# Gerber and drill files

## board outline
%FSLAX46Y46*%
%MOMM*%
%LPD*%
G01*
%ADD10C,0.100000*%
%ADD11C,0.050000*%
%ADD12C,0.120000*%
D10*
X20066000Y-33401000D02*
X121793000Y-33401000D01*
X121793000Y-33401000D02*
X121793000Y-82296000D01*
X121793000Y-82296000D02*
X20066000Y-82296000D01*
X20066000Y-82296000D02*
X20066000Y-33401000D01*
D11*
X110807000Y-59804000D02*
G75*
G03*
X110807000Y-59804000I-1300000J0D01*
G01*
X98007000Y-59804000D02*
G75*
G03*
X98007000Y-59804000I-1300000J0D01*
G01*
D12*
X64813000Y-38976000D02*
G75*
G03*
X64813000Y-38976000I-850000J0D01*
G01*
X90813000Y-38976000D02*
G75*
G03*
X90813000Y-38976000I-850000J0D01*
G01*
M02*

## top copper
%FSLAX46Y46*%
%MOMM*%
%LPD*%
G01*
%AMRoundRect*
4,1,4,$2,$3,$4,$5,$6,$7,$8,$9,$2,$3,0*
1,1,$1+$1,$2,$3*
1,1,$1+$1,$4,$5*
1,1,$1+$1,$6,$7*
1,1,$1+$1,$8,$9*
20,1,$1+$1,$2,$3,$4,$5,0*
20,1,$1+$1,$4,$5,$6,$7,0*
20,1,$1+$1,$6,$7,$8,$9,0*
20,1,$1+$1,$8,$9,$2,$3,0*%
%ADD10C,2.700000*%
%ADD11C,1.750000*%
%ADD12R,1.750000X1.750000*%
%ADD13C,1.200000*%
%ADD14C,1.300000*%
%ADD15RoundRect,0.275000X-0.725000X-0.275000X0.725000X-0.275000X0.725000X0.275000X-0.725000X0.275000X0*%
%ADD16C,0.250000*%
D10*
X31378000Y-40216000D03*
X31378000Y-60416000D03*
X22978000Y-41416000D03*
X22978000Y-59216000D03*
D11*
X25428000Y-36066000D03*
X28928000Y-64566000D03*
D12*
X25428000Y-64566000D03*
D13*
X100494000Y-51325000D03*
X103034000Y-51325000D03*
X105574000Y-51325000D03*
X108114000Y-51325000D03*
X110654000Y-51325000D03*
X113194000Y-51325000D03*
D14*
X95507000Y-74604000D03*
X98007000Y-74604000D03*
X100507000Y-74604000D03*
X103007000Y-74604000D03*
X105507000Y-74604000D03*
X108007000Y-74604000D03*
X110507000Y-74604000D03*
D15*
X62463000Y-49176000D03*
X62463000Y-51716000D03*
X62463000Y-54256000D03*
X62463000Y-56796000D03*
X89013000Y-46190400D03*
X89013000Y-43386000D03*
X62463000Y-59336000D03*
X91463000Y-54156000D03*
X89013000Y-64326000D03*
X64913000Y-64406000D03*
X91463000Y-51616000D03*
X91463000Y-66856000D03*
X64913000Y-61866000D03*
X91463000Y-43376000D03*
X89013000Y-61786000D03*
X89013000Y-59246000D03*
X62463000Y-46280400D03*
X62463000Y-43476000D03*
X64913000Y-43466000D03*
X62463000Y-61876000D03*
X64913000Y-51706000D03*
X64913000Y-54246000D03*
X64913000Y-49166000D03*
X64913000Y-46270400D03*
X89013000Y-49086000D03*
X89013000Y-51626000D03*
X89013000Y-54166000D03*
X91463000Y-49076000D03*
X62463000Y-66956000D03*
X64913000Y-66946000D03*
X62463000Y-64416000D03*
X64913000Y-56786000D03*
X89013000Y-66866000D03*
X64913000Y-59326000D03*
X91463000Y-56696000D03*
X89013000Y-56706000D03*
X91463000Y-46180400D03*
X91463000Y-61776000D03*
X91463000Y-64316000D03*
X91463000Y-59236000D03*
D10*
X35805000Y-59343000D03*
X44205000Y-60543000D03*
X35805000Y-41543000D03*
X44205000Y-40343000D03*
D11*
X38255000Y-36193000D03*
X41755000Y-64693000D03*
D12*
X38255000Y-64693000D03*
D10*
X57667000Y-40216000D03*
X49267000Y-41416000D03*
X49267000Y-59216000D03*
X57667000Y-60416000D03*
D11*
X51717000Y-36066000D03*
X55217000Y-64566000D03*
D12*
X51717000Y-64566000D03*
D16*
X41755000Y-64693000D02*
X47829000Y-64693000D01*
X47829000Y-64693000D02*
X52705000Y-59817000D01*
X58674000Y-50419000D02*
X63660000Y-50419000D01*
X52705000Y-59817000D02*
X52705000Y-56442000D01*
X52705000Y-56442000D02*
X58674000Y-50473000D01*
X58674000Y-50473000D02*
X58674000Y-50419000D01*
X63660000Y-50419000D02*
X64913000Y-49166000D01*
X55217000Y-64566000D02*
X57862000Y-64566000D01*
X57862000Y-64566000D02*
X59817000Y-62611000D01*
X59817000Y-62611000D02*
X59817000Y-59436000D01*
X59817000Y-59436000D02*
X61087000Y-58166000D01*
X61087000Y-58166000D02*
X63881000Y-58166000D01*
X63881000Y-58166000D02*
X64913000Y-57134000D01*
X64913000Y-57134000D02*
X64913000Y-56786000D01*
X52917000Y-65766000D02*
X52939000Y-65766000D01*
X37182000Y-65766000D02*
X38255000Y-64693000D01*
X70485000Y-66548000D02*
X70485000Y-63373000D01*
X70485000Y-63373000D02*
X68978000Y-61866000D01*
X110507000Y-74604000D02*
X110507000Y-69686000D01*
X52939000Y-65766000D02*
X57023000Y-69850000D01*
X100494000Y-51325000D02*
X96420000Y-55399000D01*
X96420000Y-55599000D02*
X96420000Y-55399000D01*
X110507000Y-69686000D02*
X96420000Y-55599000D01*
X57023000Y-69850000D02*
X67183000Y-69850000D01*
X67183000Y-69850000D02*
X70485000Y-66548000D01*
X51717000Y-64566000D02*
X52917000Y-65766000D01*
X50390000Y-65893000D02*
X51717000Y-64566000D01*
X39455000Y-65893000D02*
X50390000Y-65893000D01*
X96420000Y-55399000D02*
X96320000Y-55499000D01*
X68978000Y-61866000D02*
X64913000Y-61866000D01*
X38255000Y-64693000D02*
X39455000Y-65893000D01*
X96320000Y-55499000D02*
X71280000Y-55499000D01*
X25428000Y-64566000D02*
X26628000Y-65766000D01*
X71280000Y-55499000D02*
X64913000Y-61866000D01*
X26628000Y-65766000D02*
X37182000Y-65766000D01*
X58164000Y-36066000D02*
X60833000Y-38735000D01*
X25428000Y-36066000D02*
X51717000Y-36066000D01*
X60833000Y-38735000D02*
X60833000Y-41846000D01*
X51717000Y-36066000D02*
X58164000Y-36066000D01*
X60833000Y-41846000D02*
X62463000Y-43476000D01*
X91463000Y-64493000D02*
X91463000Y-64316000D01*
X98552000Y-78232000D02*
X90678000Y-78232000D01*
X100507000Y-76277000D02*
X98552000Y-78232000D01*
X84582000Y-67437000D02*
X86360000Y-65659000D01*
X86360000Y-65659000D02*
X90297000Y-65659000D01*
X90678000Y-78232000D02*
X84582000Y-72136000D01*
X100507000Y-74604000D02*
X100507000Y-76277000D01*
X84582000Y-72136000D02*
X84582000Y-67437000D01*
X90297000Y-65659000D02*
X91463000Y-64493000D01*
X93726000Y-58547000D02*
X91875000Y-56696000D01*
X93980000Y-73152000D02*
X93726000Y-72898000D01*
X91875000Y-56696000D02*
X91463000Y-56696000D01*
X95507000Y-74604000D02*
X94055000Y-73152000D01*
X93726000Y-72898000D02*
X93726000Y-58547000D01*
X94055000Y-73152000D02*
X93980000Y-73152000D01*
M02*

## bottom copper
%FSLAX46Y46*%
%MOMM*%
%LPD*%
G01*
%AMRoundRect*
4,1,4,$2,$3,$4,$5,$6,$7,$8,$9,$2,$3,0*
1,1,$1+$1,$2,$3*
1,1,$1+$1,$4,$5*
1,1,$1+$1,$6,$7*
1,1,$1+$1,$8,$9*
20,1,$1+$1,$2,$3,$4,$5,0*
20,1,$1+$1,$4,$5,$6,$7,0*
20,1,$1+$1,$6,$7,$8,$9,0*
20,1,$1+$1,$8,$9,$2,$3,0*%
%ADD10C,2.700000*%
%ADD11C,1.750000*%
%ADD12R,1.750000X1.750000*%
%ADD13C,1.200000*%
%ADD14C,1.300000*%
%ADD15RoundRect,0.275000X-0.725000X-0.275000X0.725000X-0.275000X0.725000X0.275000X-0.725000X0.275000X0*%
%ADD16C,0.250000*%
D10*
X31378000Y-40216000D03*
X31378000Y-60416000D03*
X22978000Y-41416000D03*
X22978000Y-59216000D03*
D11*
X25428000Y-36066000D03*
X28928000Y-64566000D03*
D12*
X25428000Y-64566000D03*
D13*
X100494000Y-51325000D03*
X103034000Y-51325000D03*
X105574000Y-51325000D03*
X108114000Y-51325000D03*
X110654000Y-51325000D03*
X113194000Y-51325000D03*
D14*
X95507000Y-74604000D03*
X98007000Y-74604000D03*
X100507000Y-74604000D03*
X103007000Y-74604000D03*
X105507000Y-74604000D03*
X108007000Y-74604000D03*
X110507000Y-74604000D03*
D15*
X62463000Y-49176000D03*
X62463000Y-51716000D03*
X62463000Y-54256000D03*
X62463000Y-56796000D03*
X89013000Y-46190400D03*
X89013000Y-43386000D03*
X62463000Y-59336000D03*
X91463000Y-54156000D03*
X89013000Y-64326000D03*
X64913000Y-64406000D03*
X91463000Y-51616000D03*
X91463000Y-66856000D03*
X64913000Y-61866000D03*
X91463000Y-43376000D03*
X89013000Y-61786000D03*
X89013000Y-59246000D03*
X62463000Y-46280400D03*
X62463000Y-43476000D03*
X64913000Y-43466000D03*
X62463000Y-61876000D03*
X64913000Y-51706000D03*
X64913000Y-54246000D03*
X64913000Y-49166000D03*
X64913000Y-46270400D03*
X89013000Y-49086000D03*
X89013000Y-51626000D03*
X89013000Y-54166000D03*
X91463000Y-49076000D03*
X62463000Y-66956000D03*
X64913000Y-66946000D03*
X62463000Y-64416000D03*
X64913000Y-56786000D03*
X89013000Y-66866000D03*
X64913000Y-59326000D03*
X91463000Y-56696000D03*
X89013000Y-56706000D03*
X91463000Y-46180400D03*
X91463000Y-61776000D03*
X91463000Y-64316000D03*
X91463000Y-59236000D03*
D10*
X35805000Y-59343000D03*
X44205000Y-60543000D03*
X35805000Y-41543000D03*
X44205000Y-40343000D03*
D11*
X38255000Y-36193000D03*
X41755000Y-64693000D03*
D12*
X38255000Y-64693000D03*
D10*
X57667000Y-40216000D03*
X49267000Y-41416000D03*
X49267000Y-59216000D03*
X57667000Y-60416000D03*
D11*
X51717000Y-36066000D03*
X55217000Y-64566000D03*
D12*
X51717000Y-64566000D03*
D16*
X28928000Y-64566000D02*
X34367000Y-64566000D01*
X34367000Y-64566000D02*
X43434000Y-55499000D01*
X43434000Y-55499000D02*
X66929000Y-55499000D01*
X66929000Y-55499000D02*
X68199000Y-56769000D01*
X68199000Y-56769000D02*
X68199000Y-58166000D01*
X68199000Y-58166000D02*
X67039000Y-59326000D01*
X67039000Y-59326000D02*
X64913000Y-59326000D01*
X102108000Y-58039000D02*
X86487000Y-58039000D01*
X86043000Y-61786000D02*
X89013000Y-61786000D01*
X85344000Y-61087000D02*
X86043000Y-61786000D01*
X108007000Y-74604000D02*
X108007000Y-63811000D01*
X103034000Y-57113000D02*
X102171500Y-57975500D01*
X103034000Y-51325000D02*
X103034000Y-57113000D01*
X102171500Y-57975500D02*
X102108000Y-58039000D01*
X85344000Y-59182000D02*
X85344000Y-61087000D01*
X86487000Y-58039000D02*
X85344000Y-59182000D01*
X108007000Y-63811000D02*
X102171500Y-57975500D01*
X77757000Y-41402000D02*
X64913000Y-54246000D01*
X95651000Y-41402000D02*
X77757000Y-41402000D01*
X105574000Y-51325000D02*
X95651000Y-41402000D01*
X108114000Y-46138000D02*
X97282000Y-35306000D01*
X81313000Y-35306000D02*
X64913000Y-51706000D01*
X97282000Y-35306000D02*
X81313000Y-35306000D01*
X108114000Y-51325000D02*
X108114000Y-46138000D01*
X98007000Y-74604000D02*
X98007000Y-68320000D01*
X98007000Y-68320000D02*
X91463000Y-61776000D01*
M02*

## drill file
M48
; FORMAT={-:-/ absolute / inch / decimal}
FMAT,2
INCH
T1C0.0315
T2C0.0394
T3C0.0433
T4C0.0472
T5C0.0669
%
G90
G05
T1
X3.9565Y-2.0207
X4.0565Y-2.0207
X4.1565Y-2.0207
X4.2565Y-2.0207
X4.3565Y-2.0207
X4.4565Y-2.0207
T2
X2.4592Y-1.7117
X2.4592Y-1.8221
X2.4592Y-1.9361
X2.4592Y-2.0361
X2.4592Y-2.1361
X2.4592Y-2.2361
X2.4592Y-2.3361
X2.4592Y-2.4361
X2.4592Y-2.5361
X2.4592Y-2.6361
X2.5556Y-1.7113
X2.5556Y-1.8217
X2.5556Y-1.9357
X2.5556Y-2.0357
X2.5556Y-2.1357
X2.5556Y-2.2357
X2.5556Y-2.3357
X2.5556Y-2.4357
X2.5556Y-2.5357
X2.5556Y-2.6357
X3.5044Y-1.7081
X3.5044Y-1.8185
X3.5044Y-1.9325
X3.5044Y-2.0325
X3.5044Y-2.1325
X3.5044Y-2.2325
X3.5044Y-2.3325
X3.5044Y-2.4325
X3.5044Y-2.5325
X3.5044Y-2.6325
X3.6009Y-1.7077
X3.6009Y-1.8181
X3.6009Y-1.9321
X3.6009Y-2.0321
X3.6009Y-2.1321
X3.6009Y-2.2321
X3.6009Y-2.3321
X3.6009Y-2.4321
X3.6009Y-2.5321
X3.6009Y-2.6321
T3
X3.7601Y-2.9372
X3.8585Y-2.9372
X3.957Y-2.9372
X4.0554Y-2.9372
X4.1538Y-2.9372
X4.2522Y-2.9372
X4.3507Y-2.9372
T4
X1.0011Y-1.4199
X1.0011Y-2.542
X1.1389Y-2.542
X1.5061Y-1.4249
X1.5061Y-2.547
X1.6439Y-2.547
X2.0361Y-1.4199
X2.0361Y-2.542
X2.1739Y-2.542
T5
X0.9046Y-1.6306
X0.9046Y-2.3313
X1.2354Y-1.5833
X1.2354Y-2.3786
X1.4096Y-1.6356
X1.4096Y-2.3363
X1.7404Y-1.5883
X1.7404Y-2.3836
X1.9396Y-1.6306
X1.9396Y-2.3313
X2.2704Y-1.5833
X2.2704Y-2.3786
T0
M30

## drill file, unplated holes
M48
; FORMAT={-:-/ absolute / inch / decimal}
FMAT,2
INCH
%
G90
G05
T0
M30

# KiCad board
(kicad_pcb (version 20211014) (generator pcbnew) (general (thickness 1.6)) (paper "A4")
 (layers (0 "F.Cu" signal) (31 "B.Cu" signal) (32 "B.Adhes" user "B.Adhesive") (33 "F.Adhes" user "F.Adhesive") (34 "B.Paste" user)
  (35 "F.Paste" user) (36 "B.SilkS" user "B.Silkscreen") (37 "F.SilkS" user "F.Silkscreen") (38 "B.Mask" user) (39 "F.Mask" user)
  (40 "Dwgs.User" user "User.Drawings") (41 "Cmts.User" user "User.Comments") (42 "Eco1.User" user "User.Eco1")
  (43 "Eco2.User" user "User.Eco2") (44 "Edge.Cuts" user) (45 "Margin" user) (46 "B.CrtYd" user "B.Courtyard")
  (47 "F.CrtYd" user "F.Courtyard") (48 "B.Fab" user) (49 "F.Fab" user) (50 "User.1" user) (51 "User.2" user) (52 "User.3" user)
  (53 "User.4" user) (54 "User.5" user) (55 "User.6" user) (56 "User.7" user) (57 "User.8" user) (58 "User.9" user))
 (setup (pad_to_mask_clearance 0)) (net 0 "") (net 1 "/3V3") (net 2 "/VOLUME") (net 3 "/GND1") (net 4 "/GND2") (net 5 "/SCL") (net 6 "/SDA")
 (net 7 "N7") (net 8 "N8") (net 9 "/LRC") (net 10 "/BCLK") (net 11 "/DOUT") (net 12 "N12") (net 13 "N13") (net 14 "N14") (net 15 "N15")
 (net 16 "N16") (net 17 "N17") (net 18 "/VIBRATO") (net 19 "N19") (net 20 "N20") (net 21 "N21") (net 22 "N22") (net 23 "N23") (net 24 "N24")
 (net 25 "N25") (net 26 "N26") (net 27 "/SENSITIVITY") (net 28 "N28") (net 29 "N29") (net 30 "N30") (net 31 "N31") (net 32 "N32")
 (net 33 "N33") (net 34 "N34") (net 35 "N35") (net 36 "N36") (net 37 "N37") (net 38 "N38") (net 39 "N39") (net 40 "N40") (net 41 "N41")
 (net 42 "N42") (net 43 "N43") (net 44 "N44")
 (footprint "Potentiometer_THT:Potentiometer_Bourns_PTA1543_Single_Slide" (layer "F.Cu") (at 25.428 64.566 90)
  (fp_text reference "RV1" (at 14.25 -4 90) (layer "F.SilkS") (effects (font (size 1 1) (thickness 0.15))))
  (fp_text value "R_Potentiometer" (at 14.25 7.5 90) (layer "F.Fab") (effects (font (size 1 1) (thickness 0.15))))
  (pad "1" thru_hole rect (at 0 0 90) (size 1.75 1.75) (drill 1.2) (layers *.Cu *.Mask) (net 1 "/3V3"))
  (pad "2" thru_hole circle (at 0 3.5 90) (size 1.75 1.75) (drill 1.2) (layers *.Cu *.Mask) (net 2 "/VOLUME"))
  (pad "3" thru_hole circle (at 28.5 0 90) (size 1.75 1.75) (drill 1.2) (layers *.Cu *.Mask) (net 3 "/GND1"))
  (pad "MP" thru_hole circle (at 5.35 -2.45 90) (size 2.7 2.7) (drill 1.7) (layers *.Cu *.Mask))
  (pad "MP" thru_hole circle (at 23.15 -2.45 90) (size 2.7 2.7) (drill 1.7) (layers *.Cu *.Mask))
  (pad "MP" thru_hole circle (at 4.15 5.95 90) (size 2.7 2.7) (drill 1.7) (layers *.Cu *.Mask))
  (pad "MP" thru_hole circle (at 24.35 5.95 90) (size 2.7 2.7) (drill 1.7) (layers *.Cu *.Mask)))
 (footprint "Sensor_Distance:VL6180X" (layer "F.Cu") (at 94.144 36.085)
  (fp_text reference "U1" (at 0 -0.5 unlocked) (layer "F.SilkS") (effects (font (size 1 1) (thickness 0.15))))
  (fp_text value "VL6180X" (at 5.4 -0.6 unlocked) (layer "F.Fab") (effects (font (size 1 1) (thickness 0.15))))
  (pad "1" thru_hole circle (at 6.35 15.24) (size 1.2 1.2) (drill 0.8) (layers *.Cu *.Mask) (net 1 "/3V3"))
  (pad "2" thru_hole circle (at 8.89 15.24) (size 1.2 1.2) (drill 0.8) (layers *.Cu *.Mask) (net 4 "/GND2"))
  (pad "3" thru_hole circle (at 11.43 15.24) (size 1.2 1.2) (drill 0.8) (layers *.Cu *.Mask) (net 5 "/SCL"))
  (pad "4" thru_hole circle (at 13.97 15.24) (size 1.2 1.2) (drill 0.8) (layers *.Cu *.Mask) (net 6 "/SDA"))
  (pad "5" thru_hole circle (at 16.51 15.24) (size 1.2 1.2) (drill 0.8) (layers *.Cu *.Mask) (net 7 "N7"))
  (pad "6" thru_hole circle (at 19.05 15.24) (size 1.2 1.2) (drill 0.8) (layers *.Cu *.Mask) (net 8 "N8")))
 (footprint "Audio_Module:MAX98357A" (layer "F.Cu") (at 94.107 57.404)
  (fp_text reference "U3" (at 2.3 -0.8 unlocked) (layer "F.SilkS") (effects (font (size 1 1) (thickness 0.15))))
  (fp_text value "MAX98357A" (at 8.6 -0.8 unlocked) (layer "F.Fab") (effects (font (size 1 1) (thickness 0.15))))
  (fp_circle (center 15.4 2.4) (end 16.7 2.4) (layer "Edge.Cuts") (width 0.05) (fill none))
  (fp_circle (center 2.6 2.4) (end 3.9 2.4) (layer "Edge.Cuts") (width 0.05) (fill none))
  (pad "1" thru_hole circle (at 1.4 17.2) (size 1.3 1.3) (drill 1.1) (layers *.Cu *.Mask) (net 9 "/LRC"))
  (pad "2" thru_hole circle (at 3.9 17.2) (size 1.3 1.3) (drill 1.1) (layers *.Cu *.Mask) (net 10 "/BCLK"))
  (pad "3" thru_hole circle (at 6.4 17.2) (size 1.3 1.3) (drill 1.1) (layers *.Cu *.Mask) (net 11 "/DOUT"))
  (pad "4" thru_hole circle (at 8.9 17.2) (size 1.3 1.3) (drill 1.1) (layers *.Cu *.Mask) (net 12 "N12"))
  (pad "5" thru_hole circle (at 11.4 17.2) (size 1.3 1.3) (drill 1.1) (layers *.Cu *.Mask) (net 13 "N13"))
  (pad "6" thru_hole circle (at 13.9 17.2) (size 1.3 1.3) (drill 1.1) (layers *.Cu *.Mask) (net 4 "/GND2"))
  (pad "7" thru_hole circle (at 16.4 17.2) (size 1.3 1.3) (drill 1.1) (layers *.Cu *.Mask) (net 1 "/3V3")))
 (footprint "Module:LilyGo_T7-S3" (layer "F.Cu") (at 61.463 36.476)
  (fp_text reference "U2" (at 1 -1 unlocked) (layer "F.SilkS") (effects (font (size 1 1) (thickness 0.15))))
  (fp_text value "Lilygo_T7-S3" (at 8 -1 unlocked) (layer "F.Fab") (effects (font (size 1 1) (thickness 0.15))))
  (fp_circle (center 28.5 2.5) (end 29.35 2.5) (layer "Edge.Cuts") (width 0.12) (fill none))
  (fp_circle (center 2.5 2.5) (end 3.35 2.5) (layer "Edge.Cuts") (width 0.12) (fill none))
  (pad "0" thru_hole roundrect (at 30 22.76) (size 2 1.1) (drill 1) (layers *.Cu *.Mask) (roundrect_rratio 0.25) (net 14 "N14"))
  (pad "1" thru_hole roundrect (at 30 27.84) (size 2 1.1) (drill 1) (layers *.Cu *.Mask) (roundrect_rratio 0.25) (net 11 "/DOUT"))
  (pad "2" thru_hole roundrect (at 30 25.3) (size 2 1.1) (drill 1) (layers *.Cu *.Mask) (roundrect_rratio 0.25) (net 10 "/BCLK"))
  (pad "3" thru_hole roundrect (at 30 9.7044) (size 2 1.1) (drill 1) (layers *.Cu *.Mask) (roundrect_rratio 0.25) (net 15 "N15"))
  (pad "3-1" thru_hole roundrect (at 27.55 20.23) (size 2 1.1) (drill 1) (layers *.Cu *.Mask) (roundrect_rratio 0.25) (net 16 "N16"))
  (pad "4" thru_hole roundrect (at 30 20.22) (size 2 1.1) (drill 1) (layers *.Cu *.Mask) (roundrect_rratio 0.25) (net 9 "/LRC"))
  (pad "05" thru_hole roundrect (at 3.45 22.85) (size 2 1.1) (drill 1) (layers *.Cu *.Mask) (roundrect_rratio 0.25) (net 2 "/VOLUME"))
  (pad "7" thru_hole roundrect (at 27.55 30.39) (size 2 1.1) (drill 1) (layers *.Cu *.Mask) (roundrect_rratio 0.25) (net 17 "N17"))
  (pad "08" thru_hole roundrect (at 3.45 20.31) (size 2 1.1) (drill 1) (layers *.Cu *.Mask) (roundrect_rratio 0.25) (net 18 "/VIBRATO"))
  (pad "09" thru_hole roundrect (at 1 27.94) (size 2 1.1) (drill 1) (layers *.Cu *.Mask) (roundrect_rratio 0.25) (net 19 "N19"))
  (pad "10" thru_hole roundrect (at 3.45 30.47) (size 2 1.1) (drill 1) (layers *.Cu *.Mask) (roundrect_rratio 0.25) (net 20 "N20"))
  (pad "11" thru_hole roundrect (at 1 30.48) (size 2 1.1) (drill 1) (layers *.Cu *.Mask) (roundrect_rratio 0.25) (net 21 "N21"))
  (pad "12" thru_hole roundrect (at 30 12.6) (size 2 1.1) (drill 1) (layers *.Cu *.Mask) (roundrect_rratio 0.25) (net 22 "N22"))
  (pad "12-1" thru_hole roundrect (at 27.55 17.69) (size 2 1.1) (drill 1) (layers *.Cu *.Mask) (roundrect_rratio 0.25) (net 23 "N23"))
  (pad "13" thru_hole roundrect (at 27.55 15.15) (size 2 1.1) (drill 1) (layers *.Cu *.Mask) (roundrect_rratio 0.25) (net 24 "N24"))
  (pad "14" thru_hole roundrect (at 27.55 12.61) (size 2 1.1) (drill 1) (layers *.Cu *.Mask) (roundrect_rratio 0.25) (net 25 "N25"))
  (pad "15" thru_hole roundrect (at 3.45 9.7944) (size 2 1.1) (drill 1) (layers *.Cu *.Mask) (roundrect_rratio 0.25) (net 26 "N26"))
  (pad "16" thru_hole roundrect (at 3.45 12.69) (size 2 1.1) (drill 1) (layers *.Cu *.Mask) (roundrect_rratio 0.25) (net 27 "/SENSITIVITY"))
  (pad "17" thru_hole roundrect (at 3.45 17.77) (size 2 1.1) (drill 1) (layers *.Cu *.Mask) (roundrect_rratio 0.25) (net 5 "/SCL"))
  (pad "18" thru_hole roundrect (at 3.45 15.23) (size 2 1.1) (drill 1) (layers *.Cu *.Mask) (roundrect_rratio 0.25) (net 6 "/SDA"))
  (pad "21" thru_hole roundrect (at 1 25.4) (size 2 1.1) (drill 1) (layers *.Cu *.Mask) (roundrect_rratio 0.25) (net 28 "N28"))
  (pad "30" thru_hole roundrect (at 3.45 6.99) (size 2 1.1) (drill 1) (layers *.Cu *.Mask) (roundrect_rratio 0.25) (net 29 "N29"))
  (pad "31" thru_hole roundrect (at 1 7) (size 2 1.1) (drill 1) (layers *.Cu *.Mask) (roundrect_rratio 0.25) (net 3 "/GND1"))
  (pad "32" thru_hole roundrect (at 1 9.8044) (size 2 1.1) (drill 1) (layers *.Cu *.Mask) (roundrect_rratio 0.25) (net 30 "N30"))
  (pad "33" thru_hole roundrect (at 27.55 22.77) (size 2 1.1) (drill 1) (layers *.Cu *.Mask) (roundrect_rratio 0.25) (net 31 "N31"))
  (pad "34" thru_hole roundrect (at 27.55 25.31) (size 2 1.1) (drill 1) (layers *.Cu *.Mask) (roundrect_rratio 0.25) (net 4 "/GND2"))
  (pad "35" thru_hole roundrect (at 30 6.9) (size 2 1.1) (drill 1) (layers *.Cu *.Mask) (roundrect_rratio 0.25) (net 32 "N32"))
  (pad "36" thru_hole roundrect (at 3.45 25.39) (size 2 1.1) (drill 1) (layers *.Cu *.Mask) (roundrect_rratio 0.25) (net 1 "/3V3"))
  (pad "37" thru_hole roundrect (at 30 30.38) (size 2 1.1) (drill 1) (layers *.Cu *.Mask) (roundrect_rratio 0.25) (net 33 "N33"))
  (pad "38" thru_hole roundrect (at 30 15.14) (size 2 1.1) (drill 1) (layers *.Cu *.Mask) (roundrect_rratio 0.25) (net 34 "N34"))
  (pad "39" thru_hole roundrect (at 3.45 27.93) (size 2 1.1) (drill 1) (layers *.Cu *.Mask) (roundrect_rratio 0.25) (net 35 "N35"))
  (pad "40" thru_hole roundrect (at 27.55 27.85) (size 2 1.1) (drill 1) (layers *.Cu *.Mask) (roundrect_rratio 0.25) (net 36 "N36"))
  (pad "41" thru_hole roundrect (at 30 17.68) (size 2 1.1) (drill 1) (layers *.Cu *.Mask) (roundrect_rratio 0.25) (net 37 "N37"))
  (pad "42" thru_hole roundrect (at 1 22.86) (size 2 1.1) (drill 1) (layers *.Cu *.Mask) (roundrect_rratio 0.25) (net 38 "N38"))
  (pad "43" thru_hole roundrect (at 27.55 6.91) (size 2 1.1) (drill 1) (layers *.Cu *.Mask) (roundrect_rratio 0.25) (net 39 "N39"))
  (pad "44" thru_hole roundrect (at 27.55 9.7144) (size 2 1.1) (drill 1) (layers *.Cu *.Mask) (roundrect_rratio 0.25) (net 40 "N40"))
  (pad "45" thru_hole roundrect (at 1 20.32) (size 2 1.1) (drill 1) (layers *.Cu *.Mask) (roundrect_rratio 0.25) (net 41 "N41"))
  (pad "46" thru_hole roundrect (at 1 17.78) (size 2 1.1) (drill 1) (layers *.Cu *.Mask) (roundrect_rratio 0.25) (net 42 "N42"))
  (pad "47" thru_hole roundrect (at 1 15.24) (size 2 1.1) (drill 1) (layers *.Cu *.Mask) (roundrect_rratio 0.25) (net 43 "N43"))
  (pad "48" thru_hole roundrect (at 1 12.7) (size 2 1.1) (drill 1) (layers *.Cu *.Mask) (roundrect_rratio 0.25) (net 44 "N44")))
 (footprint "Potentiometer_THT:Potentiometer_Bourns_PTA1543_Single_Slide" (layer "F.Cu") (at 38.255 64.693 90)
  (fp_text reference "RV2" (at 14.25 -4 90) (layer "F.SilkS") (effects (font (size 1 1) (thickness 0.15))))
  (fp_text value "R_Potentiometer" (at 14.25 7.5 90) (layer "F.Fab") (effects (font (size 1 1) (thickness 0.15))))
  (pad "1" thru_hole rect (at 0 0 90) (size 1.75 1.75) (drill 1.2) (layers *.Cu *.Mask) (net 1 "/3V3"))
  (pad "2" thru_hole circle (at 0 3.5 90) (size 1.75 1.75) (drill 1.2) (layers *.Cu *.Mask) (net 27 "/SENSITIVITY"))
  (pad "3" thru_hole circle (at 28.5 0 90) (size 1.75 1.75) (drill 1.2) (layers *.Cu *.Mask) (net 3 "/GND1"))
  (pad "MP" thru_hole circle (at 24.35 5.95 90) (size 2.7 2.7) (drill 1.7) (layers *.Cu *.Mask))
  (pad "MP" thru_hole circle (at 23.15 -2.45 90) (size 2.7 2.7) (drill 1.7) (layers *.Cu *.Mask))
  (pad "MP" thru_hole circle (at 4.15 5.95 90) (size 2.7 2.7) (drill 1.7) (layers *.Cu *.Mask))
  (pad "MP" thru_hole circle (at 5.35 -2.45 90) (size 2.7 2.7) (drill 1.7) (layers *.Cu *.Mask)))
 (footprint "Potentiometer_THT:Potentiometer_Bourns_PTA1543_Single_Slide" (layer "F.Cu") (at 51.717 64.566 90)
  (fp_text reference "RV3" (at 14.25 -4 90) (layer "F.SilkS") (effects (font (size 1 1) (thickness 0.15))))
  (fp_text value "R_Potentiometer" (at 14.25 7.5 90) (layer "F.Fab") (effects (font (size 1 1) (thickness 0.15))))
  (pad "1" thru_hole rect (at 0 0 90) (size 1.75 1.75) (drill 1.2) (layers *.Cu *.Mask) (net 1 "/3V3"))
  (pad "2" thru_hole circle (at 0 3.5 90) (size 1.75 1.75) (drill 1.2) (layers *.Cu *.Mask) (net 18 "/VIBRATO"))
  (pad "3" thru_hole circle (at 28.5 0 90) (size 1.75 1.75) (drill 1.2) (layers *.Cu *.Mask) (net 3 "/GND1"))
  (pad "MP" thru_hole circle (at 4.15 5.95 90) (size 2.7 2.7) (drill 1.7) (layers *.Cu *.Mask))
  (pad "MP" thru_hole circle (at 5.35 -2.45 90) (size 2.7 2.7) (drill 1.7) (layers *.Cu *.Mask))
  (pad "MP" thru_hole circle (at 23.15 -2.45 90) (size 2.7 2.7) (drill 1.7) (layers *.Cu *.Mask))
  (pad "MP" thru_hole circle (at 24.35 5.95 90) (size 2.7 2.7) (drill 1.7) (layers *.Cu *.Mask)))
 (gr_rect (start 20.066 33.401) (end 121.793 82.296) (layer "Edge.Cuts") (width 0.1) (fill none))
 (segment (start 52.917 65.766) (end 52.939 65.766) (width 0.25) (layer "F.Cu") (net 1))
 (segment (start 37.182 65.766) (end 38.255 64.693) (width 0.25) (layer "F.Cu") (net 1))
 (segment (start 70.485 66.548) (end 70.485 63.373) (width 0.25) (layer "F.Cu") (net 1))
 (segment (start 70.485 63.373) (end 68.978 61.866) (width 0.25) (layer "F.Cu") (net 1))
 (segment (start 110.507 74.604) (end 110.507 69.686) (width 0.25) (layer "F.Cu") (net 1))
 (segment (start 52.939 65.766) (end 57.023 69.85) (width 0.25) (layer "F.Cu") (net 1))
 (segment (start 100.494 51.325) (end 96.42 55.399) (width 0.25) (layer "F.Cu") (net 1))
 (segment (start 96.42 55.599) (end 96.42 55.399) (width 0.25) (layer "F.Cu") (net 1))
 (segment (start 110.507 69.686) (end 96.42 55.599) (width 0.25) (layer "F.Cu") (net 1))
 (segment (start 57.023 69.85) (end 67.183 69.85) (width 0.25) (layer "F.Cu") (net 1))
 (segment (start 67.183 69.85) (end 70.485 66.548) (width 0.25) (layer "F.Cu") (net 1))
 (segment (start 51.717 64.566) (end 52.917 65.766) (width 0.25) (layer "F.Cu") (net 1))
 (segment (start 50.39 65.893) (end 51.717 64.566) (width 0.25) (layer "F.Cu") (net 1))
 (segment (start 39.455 65.893) (end 50.39 65.893) (width 0.25) (layer "F.Cu") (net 1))
 (segment (start 96.42 55.399) (end 96.32 55.499) (width 0.25) (layer "F.Cu") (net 1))
 (segment (start 68.978 61.866) (end 64.913 61.866) (width 0.25) (layer "F.Cu") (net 1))
 (segment (start 38.255 64.693) (end 39.455 65.893) (width 0.25) (layer "F.Cu") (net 1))
 (segment (start 96.32 55.499) (end 71.28 55.499) (width 0.25) (layer "F.Cu") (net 1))
 (segment (start 25.428 64.566) (end 26.628 65.766) (width 0.25) (layer "F.Cu") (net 1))
 (segment (start 71.28 55.499) (end 64.913 61.866) (width 0.25) (layer "F.Cu") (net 1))
 (segment (start 26.628 65.766) (end 37.182 65.766) (width 0.25) (layer "F.Cu") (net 1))
 (segment (start 68.199 58.166) (end 67.039 59.326) (width 0.25) (layer "B.Cu") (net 2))
 (segment (start 28.928 64.566) (end 34.367 64.566) (width 0.25) (layer "B.Cu") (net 2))
 (segment (start 67.039 59.326) (end 64.913 59.326) (width 0.25) (layer "B.Cu") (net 2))
 (segment (start 66.929 55.499) (end 68.199 56.769) (width 0.25) (layer "B.Cu") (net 2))
 (segment (start 43.434 55.499) (end 66.929 55.499) (width 0.25) (layer "B.Cu") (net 2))
 (segment (start 34.367 64.566) (end 43.434 55.499) (width 0.25) (layer "B.Cu") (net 2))
 (segment (start 68.199 56.769) (end 68.199 58.166) (width 0.25) (layer "B.Cu") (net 2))
 (segment (start 58.164 36.066) (end 60.833 38.735) (width 0.25) (layer "F.Cu") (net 3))
 (segment (start 25.428 36.066) (end 51.717 36.066) (width 0.25) (layer "F.Cu") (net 3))
 (segment (start 60.833 38.735) (end 60.833 41.846) (width 0.25) (layer "F.Cu") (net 3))
 (segment (start 51.717 36.066) (end 58.164 36.066) (width 0.25) (layer "F.Cu") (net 3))
 (segment (start 60.833 41.846) (end 62.463 43.476) (width 0.25) (layer "F.Cu") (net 3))
 (segment (start 52.705 56.442) (end 58.674 50.473) (width 0.25) (layer "F.Cu") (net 27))
 (segment (start 47.829 64.693) (end 52.705 59.817) (width 0.25) (layer "F.Cu") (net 27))
 (segment (start 41.755 64.693) (end 47.829 64.693) (width 0.25) (layer "F.Cu") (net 27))
 (segment (start 58.674 50.419) (end 63.66 50.419) (width 0.25) (layer "F.Cu") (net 27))
 (segment (start 58.674 50.473) (end 58.674 50.419) (width 0.25) (layer "F.Cu") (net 27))
 (segment (start 52.705 59.817) (end 52.705 56.442) (width 0.25) (layer "F.Cu") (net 27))
 (segment (start 63.66 50.419) (end 64.913 49.166) (width 0.25) (layer "F.Cu") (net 27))
 (segment (start 55.217 64.566) (end 57.862 64.566) (width 0.25) (layer "F.Cu") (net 18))
 (segment (start 59.817 59.436) (end 61.087 58.166) (width 0.25) (layer "F.Cu") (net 18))
 (segment (start 57.862 64.566) (end 59.817 62.611) (width 0.25) (layer "F.Cu") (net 18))
 (segment (start 59.817 62.611) (end 59.817 59.436) (width 0.25) (layer "F.Cu") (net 18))
 (segment (start 61.087 58.166) (end 63.881 58.166) (width 0.25) (layer "F.Cu") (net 18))
 (segment (start 64.913 57.134) (end 64.913 56.786) (width 0.25) (layer "F.Cu") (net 18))
 (segment (start 63.881 58.166) (end 64.913 57.134) (width 0.25) (layer "F.Cu") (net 18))
 (segment (start 102.108 58.039) (end 86.487 58.039) (width 0.25) (layer "B.Cu") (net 4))
 (segment (start 86.043 61.786) (end 89.013 61.786) (width 0.25) (layer "B.Cu") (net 4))
 (segment (start 85.344 61.087) (end 86.043 61.786) (width 0.25) (layer "B.Cu") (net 4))
 (segment (start 108.007 74.604) (end 108.007 63.811) (width 0.25) (layer "B.Cu") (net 4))
 (segment (start 103.034 57.113) (end 102.1715 57.9755) (width 0.25) (layer "B.Cu") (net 4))
 (segment (start 103.034 51.325) (end 103.034 57.113) (width 0.25) (layer "B.Cu") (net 4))
 (segment (start 102.1715 57.9755) (end 102.108 58.039) (width 0.25) (layer "B.Cu") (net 4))
 (segment (start 85.344 59.182) (end 85.344 61.087) (width 0.25) (layer "B.Cu") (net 4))
 (segment (start 86.487 58.039) (end 85.344 59.182) (width 0.25) (layer "B.Cu") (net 4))
 (segment (start 108.007 63.811) (end 102.1715 57.9755) (width 0.25) (layer "B.Cu") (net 4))
 (segment (start 77.757 41.402) (end 64.913 54.246) (width 0.25) (layer "B.Cu") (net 5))
 (segment (start 95.651 41.402) (end 77.757 41.402) (width 0.25) (layer "B.Cu") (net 5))
 (segment (start 105.574 51.325) (end 95.651 41.402) (width 0.25) (layer "B.Cu") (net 5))
 (segment (start 108.114 46.138) (end 97.282 35.306) (width 0.25) (layer "B.Cu") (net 6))
 (segment (start 81.313 35.306) (end 64.913 51.706) (width 0.25) (layer "B.Cu") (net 6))
 (segment (start 97.282 35.306) (end 81.313 35.306) (width 0.25) (layer "B.Cu") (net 6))
 (segment (start 108.114 51.325) (end 108.114 46.138) (width 0.25) (layer "B.Cu") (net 6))
 (segment (start 91.463 64.493) (end 91.463 64.316) (width 0.25) (layer "F.Cu") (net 11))
 (segment (start 98.552 78.232) (end 90.678 78.232) (width 0.25) (layer "F.Cu") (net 11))
 (segment (start 100.507 76.277) (end 98.552 78.232) (width 0.25) (layer "F.Cu") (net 11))
 (segment (start 84.582 67.437) (end 86.36 65.659) (width 0.25) (layer "F.Cu") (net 11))
 (segment (start 86.36 65.659) (end 90.297 65.659) (width 0.25) (layer "F.Cu") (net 11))
 (segment (start 90.678 78.232) (end 84.582 72.136) (width 0.25) (layer "F.Cu") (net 11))
 (segment (start 100.507 74.604) (end 100.507 76.277) (width 0.25) (layer "F.Cu") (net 11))
 (segment (start 84.582 72.136) (end 84.582 67.437) (width 0.25) (layer "F.Cu") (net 11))
 (segment (start 90.297 65.659) (end 91.463 64.493) (width 0.25) (layer "F.Cu") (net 11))
 (segment (start 98.007 74.604) (end 98.007 68.32) (width 0.25) (layer "B.Cu") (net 10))
 (segment (start 98.007 68.32) (end 91.463 61.776) (width 0.25) (layer "B.Cu") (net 10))
 (segment (start 93.726 58.547) (end 91.875 56.696) (width 0.25) (layer "F.Cu") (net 9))
 (segment (start 93.98 73.152) (end 93.726 72.898) (width 0.25) (layer "F.Cu") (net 9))
 (segment (start 91.875 56.696) (end 91.463 56.696) (width 0.25) (layer "F.Cu") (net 9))
 (segment (start 95.507 74.604) (end 94.055 73.152) (width 0.25) (layer "F.Cu") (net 9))
 (segment (start 93.726 72.898) (end 93.726 58.547) (width 0.25) (layer "F.Cu") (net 9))
 (segment (start 94.055 73.152) (end 93.98 73.152) (width 0.25) (layer "F.Cu") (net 9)))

